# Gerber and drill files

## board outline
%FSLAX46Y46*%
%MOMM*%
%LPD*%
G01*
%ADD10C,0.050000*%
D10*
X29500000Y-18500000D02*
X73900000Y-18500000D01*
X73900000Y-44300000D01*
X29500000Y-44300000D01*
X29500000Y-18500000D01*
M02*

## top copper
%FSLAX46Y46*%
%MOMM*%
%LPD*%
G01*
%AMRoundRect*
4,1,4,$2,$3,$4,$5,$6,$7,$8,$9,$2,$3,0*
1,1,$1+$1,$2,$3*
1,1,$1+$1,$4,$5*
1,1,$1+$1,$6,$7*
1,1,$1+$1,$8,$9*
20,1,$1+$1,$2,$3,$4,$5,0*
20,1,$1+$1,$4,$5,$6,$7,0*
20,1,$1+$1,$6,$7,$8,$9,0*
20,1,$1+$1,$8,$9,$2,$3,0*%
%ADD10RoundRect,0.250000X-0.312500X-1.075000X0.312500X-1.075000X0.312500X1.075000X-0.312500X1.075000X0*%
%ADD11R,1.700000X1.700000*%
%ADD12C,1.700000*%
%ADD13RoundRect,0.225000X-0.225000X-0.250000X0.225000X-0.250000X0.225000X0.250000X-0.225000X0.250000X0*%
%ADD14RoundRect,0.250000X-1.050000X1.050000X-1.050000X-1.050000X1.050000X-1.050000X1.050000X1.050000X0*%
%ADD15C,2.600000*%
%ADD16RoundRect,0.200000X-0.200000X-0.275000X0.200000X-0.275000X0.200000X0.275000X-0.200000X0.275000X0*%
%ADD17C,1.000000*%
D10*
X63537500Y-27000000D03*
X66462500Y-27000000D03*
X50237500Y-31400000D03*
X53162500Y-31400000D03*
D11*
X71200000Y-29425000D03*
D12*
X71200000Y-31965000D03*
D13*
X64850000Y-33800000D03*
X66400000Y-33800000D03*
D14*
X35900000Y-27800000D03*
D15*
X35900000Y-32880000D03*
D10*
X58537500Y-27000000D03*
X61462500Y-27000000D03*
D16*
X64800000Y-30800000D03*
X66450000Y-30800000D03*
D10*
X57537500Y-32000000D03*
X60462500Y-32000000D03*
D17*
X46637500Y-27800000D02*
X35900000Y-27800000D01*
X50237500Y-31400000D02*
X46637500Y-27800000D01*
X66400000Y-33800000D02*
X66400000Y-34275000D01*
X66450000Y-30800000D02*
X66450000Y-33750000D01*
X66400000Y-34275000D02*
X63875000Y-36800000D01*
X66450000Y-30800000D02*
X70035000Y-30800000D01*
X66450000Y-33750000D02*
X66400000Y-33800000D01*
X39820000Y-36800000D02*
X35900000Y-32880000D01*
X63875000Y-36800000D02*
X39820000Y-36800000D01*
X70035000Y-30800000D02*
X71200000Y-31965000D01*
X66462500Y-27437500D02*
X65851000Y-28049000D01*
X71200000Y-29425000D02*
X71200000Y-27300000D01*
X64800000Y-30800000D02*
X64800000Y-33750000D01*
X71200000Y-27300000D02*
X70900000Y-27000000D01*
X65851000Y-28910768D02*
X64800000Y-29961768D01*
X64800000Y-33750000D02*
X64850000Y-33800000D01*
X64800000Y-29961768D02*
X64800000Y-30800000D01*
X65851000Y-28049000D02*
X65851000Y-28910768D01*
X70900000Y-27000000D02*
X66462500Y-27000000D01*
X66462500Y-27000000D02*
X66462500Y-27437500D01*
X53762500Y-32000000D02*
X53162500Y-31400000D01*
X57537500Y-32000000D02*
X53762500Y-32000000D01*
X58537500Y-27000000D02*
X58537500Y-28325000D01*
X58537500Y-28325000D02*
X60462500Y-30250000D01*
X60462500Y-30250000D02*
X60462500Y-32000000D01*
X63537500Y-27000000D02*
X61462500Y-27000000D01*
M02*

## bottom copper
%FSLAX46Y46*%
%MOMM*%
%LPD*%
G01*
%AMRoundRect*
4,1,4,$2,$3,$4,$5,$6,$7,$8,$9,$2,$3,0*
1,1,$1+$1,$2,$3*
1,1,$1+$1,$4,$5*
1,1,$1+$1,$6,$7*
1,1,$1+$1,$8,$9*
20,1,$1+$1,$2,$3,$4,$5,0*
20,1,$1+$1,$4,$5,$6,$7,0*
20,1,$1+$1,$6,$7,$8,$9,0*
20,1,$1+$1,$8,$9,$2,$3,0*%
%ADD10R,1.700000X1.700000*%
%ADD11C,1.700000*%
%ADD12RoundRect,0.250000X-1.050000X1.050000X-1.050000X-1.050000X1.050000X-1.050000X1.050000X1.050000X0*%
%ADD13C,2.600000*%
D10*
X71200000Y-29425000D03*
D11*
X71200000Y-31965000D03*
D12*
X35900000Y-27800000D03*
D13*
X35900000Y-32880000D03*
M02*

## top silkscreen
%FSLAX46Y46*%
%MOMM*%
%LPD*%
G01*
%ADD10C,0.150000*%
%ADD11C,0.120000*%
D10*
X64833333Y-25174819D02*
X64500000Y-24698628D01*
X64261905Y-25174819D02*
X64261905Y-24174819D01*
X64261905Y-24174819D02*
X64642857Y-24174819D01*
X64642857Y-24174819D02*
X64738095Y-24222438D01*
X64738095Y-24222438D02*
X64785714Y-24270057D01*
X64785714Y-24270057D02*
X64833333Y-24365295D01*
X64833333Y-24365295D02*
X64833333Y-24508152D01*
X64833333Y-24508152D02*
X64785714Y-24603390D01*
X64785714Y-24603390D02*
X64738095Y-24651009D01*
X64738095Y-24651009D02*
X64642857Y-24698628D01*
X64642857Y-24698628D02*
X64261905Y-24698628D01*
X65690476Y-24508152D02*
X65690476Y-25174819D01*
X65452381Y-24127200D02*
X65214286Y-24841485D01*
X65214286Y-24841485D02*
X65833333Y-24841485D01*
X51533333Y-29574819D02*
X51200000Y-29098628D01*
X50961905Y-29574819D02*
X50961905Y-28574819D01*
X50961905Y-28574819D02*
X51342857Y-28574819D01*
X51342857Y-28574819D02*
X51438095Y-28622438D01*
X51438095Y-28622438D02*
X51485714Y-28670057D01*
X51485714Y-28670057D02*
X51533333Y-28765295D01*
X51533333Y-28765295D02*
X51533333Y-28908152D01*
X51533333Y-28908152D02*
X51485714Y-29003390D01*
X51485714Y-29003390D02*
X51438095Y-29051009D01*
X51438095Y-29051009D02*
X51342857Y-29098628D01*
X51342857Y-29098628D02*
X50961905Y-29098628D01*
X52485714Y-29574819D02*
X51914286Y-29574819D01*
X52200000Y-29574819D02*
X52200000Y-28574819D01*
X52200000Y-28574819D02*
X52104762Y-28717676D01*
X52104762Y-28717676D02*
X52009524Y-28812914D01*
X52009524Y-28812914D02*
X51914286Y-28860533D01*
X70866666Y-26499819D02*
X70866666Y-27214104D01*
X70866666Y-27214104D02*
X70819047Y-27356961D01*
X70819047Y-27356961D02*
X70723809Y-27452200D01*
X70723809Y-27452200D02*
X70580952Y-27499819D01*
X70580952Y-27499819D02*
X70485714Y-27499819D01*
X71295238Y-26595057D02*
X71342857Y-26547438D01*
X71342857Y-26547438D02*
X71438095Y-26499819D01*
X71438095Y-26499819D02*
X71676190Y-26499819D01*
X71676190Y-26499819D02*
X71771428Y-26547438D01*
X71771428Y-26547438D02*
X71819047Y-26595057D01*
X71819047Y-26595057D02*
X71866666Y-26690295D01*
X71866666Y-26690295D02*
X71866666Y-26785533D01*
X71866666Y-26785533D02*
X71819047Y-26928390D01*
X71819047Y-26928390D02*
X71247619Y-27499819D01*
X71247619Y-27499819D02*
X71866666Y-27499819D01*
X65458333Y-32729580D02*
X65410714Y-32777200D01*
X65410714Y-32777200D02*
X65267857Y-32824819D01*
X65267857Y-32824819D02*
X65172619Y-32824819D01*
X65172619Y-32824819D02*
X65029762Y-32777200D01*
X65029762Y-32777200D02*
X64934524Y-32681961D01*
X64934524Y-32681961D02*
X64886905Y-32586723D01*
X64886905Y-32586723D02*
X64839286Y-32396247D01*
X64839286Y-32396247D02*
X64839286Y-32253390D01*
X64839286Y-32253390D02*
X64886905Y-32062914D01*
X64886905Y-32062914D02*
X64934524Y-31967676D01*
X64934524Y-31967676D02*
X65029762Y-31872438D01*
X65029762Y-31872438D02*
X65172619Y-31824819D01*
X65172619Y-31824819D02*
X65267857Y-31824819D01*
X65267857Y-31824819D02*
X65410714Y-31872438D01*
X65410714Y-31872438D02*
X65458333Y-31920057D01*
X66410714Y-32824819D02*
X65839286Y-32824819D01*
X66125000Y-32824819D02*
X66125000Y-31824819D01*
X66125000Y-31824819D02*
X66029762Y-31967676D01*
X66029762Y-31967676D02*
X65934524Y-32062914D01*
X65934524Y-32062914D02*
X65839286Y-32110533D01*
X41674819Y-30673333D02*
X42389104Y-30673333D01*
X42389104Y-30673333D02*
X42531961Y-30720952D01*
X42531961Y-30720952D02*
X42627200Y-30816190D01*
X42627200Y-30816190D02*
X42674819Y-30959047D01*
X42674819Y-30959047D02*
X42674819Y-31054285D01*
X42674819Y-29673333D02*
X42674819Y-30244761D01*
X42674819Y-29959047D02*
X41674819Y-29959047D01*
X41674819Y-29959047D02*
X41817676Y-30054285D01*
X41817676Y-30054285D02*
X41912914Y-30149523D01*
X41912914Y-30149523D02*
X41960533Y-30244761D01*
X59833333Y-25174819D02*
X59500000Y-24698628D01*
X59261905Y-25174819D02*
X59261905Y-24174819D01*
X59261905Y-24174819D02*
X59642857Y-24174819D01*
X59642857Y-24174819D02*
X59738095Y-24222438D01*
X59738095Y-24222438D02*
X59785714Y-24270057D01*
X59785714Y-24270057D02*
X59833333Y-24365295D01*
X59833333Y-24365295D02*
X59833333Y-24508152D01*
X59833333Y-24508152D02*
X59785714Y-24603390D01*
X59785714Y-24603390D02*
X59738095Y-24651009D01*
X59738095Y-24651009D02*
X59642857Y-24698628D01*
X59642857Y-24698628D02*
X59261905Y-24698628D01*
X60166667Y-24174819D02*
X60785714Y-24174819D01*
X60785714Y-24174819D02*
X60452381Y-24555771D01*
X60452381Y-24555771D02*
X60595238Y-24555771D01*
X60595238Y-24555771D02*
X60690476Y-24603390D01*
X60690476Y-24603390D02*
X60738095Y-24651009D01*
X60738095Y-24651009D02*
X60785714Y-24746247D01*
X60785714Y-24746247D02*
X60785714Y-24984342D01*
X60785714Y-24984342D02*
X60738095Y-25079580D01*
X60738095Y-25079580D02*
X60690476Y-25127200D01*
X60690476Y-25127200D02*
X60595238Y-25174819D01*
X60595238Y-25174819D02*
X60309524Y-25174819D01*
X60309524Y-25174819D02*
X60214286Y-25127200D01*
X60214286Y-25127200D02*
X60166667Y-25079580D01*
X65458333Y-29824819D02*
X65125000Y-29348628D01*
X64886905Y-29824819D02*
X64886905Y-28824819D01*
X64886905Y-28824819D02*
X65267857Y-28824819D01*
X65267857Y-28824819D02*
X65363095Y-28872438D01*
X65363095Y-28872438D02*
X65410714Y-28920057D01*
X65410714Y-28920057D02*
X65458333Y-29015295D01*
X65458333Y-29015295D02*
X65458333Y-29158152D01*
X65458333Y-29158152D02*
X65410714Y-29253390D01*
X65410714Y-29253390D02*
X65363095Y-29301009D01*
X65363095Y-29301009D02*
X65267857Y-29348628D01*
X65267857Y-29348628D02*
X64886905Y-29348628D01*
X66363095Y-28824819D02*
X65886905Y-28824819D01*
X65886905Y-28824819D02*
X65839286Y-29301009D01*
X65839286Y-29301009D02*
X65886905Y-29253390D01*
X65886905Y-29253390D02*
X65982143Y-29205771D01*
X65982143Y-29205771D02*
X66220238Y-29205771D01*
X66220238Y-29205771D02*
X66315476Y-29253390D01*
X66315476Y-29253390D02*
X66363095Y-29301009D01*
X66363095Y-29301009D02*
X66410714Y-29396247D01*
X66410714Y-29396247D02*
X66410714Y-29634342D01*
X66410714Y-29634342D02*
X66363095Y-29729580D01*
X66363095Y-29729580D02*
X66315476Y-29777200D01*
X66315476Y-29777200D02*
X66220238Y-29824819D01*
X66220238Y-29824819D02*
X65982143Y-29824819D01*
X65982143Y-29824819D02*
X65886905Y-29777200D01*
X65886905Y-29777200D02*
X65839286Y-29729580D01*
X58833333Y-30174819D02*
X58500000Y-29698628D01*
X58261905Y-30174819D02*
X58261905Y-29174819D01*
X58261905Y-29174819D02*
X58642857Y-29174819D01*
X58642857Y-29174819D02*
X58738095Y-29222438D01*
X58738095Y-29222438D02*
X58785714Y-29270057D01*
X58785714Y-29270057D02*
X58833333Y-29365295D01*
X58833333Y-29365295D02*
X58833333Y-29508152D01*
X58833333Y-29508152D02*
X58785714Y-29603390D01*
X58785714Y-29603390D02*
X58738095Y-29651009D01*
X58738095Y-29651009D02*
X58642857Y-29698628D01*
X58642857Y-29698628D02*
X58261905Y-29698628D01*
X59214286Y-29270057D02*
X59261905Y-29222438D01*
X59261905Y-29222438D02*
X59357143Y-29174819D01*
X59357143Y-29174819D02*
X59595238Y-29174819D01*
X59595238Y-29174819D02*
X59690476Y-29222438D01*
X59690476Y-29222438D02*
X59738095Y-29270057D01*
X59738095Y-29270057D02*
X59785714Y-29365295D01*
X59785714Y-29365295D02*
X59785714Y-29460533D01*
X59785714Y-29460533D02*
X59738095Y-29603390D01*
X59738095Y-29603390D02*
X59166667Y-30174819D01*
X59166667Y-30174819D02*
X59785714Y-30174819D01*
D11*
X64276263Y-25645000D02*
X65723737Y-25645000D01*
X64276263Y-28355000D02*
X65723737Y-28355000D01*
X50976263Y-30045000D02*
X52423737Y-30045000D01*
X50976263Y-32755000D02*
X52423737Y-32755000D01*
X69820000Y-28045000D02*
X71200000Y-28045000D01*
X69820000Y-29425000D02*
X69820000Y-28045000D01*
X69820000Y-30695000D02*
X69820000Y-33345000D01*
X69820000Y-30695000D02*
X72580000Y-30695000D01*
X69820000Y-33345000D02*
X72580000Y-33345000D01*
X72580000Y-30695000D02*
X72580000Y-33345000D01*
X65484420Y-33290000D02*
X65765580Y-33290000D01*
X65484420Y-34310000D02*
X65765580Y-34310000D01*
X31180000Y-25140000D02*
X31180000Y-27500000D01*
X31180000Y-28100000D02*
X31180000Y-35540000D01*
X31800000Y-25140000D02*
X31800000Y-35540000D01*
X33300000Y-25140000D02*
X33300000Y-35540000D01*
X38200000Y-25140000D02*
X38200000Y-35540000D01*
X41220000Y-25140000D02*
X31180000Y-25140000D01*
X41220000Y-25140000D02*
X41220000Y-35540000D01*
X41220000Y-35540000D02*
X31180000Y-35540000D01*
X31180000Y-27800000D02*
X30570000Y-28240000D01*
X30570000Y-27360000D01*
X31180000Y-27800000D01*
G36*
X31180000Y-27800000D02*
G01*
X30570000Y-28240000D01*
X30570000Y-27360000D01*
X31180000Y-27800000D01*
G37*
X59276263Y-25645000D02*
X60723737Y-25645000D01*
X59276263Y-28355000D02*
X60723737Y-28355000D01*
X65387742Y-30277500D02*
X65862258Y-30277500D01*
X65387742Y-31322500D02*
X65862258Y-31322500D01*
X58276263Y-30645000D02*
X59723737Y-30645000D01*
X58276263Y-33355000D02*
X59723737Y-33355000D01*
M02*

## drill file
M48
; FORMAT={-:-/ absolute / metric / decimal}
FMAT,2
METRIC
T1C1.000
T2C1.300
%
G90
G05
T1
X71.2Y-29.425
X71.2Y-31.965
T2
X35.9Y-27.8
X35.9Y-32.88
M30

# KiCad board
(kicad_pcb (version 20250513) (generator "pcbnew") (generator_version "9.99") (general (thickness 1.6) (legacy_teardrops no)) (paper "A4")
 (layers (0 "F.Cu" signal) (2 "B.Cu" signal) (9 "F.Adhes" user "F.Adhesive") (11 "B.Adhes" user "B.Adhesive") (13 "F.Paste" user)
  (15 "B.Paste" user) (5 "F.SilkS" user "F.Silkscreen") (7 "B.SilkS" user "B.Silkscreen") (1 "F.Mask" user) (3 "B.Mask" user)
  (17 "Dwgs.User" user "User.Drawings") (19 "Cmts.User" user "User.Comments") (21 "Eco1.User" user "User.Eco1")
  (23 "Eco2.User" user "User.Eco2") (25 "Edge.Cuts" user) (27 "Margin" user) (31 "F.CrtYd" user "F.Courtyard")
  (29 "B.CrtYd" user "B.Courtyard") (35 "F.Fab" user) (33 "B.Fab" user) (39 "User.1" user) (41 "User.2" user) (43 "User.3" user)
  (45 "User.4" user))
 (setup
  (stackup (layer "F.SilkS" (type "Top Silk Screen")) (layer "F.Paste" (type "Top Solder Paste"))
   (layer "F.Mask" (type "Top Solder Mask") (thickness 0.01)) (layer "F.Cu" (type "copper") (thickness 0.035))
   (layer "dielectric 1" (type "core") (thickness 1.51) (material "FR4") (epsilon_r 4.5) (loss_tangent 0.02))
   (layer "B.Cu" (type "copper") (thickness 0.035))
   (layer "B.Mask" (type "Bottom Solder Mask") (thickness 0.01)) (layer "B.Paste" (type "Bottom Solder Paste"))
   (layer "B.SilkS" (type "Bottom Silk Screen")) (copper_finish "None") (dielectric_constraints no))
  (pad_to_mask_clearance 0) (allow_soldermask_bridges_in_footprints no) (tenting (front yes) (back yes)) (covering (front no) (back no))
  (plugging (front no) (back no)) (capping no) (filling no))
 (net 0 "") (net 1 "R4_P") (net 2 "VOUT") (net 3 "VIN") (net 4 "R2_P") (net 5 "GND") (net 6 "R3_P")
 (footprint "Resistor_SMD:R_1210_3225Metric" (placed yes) (layer "F.Cu") (at 65 27)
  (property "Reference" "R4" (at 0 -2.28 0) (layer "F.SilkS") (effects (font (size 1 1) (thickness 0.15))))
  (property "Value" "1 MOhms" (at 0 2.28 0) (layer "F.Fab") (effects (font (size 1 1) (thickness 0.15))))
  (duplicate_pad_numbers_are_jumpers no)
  (fp_line (start -0.723737 -1.355) (end 0.723737 -1.355) (stroke (width 0.12) (type solid)) (layer "F.SilkS"))
  (fp_line (start -0.723737 1.355) (end 0.723737 1.355) (stroke (width 0.12) (type solid)) (layer "F.SilkS"))
  (pad "1" smd roundrect (at -1.4625 0) (size 1.125 2.65) (layers "F.Cu" "F.Mask" "F.Paste") (roundrect_rratio 0.222222) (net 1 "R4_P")
   (tenting (front none) (back none)))
  (pad "2" smd roundrect (at 1.4625 0) (size 1.125 2.65) (layers "F.Cu" "F.Mask" "F.Paste") (roundrect_rratio 0.222222) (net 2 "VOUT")
   (tenting (front none) (back none))))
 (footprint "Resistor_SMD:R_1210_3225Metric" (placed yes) (layer "F.Cu") (at 51.7 31.4)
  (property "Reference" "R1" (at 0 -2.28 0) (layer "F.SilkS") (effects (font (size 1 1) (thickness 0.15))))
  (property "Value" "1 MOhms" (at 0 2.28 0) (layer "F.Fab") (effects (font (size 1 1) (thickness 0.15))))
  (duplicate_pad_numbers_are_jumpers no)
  (fp_line (start -0.723737 -1.355) (end 0.723737 -1.355) (stroke (width 0.12) (type solid)) (layer "F.SilkS"))
  (fp_line (start -0.723737 1.355) (end 0.723737 1.355) (stroke (width 0.12) (type solid)) (layer "F.SilkS"))
  (pad "1" smd roundrect (at -1.4625 0) (size 1.125 2.65) (layers "F.Cu" "F.Mask" "F.Paste") (roundrect_rratio 0.222222) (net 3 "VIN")
   (tenting (front none) (back none)))
  (pad "2" smd roundrect (at 1.4625 0) (size 1.125 2.65) (layers "F.Cu" "F.Mask" "F.Paste") (roundrect_rratio 0.222222) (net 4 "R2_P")
   (tenting (front none) (back none))))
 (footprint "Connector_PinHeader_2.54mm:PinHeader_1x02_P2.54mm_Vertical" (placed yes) (layer "F.Cu") (at 71.2 29.425)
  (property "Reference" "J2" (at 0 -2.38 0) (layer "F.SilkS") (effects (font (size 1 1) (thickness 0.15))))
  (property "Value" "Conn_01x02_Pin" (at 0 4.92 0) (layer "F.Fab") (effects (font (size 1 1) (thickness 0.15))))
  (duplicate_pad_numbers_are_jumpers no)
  (fp_line (start -1.38 -1.38) (end 0 -1.38) (stroke (width 0.12) (type solid)) (layer "F.SilkS"))
  (fp_line (start -1.38 0) (end -1.38 -1.38) (stroke (width 0.12) (type solid)) (layer "F.SilkS"))
  (fp_line (start -1.38 1.27) (end -1.38 3.92) (stroke (width 0.12) (type solid)) (layer "F.SilkS"))
  (fp_line (start -1.38 1.27) (end 1.38 1.27) (stroke (width 0.12) (type solid)) (layer "F.SilkS"))
  (fp_line (start -1.38 3.92) (end 1.38 3.92) (stroke (width 0.12) (type solid)) (layer "F.SilkS"))
  (fp_line (start 1.38 1.27) (end 1.38 3.92) (stroke (width 0.12) (type solid)) (layer "F.SilkS"))
  (pad "1" thru_hole rect (at 0 0) (size 1.7 1.7) (drill 1) (layers "*.Cu" "*.Mask") (remove_unused_layers no) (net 2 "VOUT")
   (tenting (front none) (back none)))
  (pad "2" thru_hole circle (at 0 2.54) (size 1.7 1.7) (drill 1) (layers "*.Cu" "*.Mask") (remove_unused_layers no) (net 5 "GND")
   (tenting (front none) (back none))))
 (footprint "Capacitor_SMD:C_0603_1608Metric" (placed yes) (layer "F.Cu") (at 65.625 33.8)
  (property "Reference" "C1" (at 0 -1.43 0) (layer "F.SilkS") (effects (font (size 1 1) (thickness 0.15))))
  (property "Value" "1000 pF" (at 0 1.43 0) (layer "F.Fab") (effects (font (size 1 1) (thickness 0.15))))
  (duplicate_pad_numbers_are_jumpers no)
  (fp_line (start -0.14058 -0.51) (end 0.14058 -0.51) (stroke (width 0.12) (type solid)) (layer "F.SilkS"))
  (fp_line (start -0.14058 0.51) (end 0.14058 0.51) (stroke (width 0.12) (type solid)) (layer "F.SilkS"))
  (pad "1" smd roundrect (at -0.775 0) (size 0.9 0.95) (layers "F.Cu" "F.Mask" "F.Paste") (roundrect_rratio 0.25) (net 2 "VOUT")
   (tenting (front none) (back none)))
  (pad "2" smd roundrect (at 0.775 0) (size 0.9 0.95) (layers "F.Cu" "F.Mask" "F.Paste") (roundrect_rratio 0.25) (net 5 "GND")
   (tenting (front none) (back none))))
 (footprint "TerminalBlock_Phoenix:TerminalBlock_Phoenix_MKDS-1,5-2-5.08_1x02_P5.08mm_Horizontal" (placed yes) (layer "F.Cu")
  (at 35.9 27.8 -90)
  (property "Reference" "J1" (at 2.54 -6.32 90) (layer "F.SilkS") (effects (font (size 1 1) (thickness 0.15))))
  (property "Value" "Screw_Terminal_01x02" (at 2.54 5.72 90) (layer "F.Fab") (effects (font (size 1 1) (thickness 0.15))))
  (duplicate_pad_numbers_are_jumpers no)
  (fp_line (start -2.66 4.72) (end -0.3 4.72) (stroke (width 0.12) (type solid)) (layer "F.SilkS"))
  (fp_line (start 0.3 4.72) (end 7.74 4.72) (stroke (width 0.12) (type solid)) (layer "F.SilkS"))
  (fp_line (start -2.66 4.1) (end 7.74 4.1) (stroke (width 0.12) (type solid)) (layer "F.SilkS"))
  (fp_line (start -2.66 2.6) (end 7.74 2.6) (stroke (width 0.12) (type solid)) (layer "F.SilkS"))
  (fp_line (start -2.66 -2.3) (end 7.74 -2.3) (stroke (width 0.12) (type solid)) (layer "F.SilkS"))
  (fp_line (start -2.66 -5.32) (end -2.66 4.72) (stroke (width 0.12) (type solid)) (layer "F.SilkS"))
  (fp_line (start -2.66 -5.32) (end 7.74 -5.32) (stroke (width 0.12) (type solid)) (layer "F.SilkS"))
  (fp_line (start 7.74 -5.32) (end 7.74 4.72) (stroke (width 0.12) (type solid)) (layer "F.SilkS"))
  (fp_poly (pts (xy 0 4.72) (xy 0.44 5.33) (xy -0.44 5.33)) (stroke (width 0.12) (type solid)) (fill yes) (layer "F.SilkS"))
  (pad "1" thru_hole roundrect (at 0 0 270) (size 2.6 2.6) (drill 1.3) (layers "*.Cu" "*.Mask") (remove_unused_layers no)
   (roundrect_rratio 0.096154) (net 3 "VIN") (tenting (front none) (back none)))
  (pad "2" thru_hole circle (at 5.08 0 270) (size 2.6 2.6) (drill 1.3) (layers "*.Cu" "*.Mask") (remove_unused_layers no) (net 5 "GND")
   (tenting (front none) (back none))))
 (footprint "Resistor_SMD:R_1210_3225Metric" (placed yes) (layer "F.Cu") (at 60 27)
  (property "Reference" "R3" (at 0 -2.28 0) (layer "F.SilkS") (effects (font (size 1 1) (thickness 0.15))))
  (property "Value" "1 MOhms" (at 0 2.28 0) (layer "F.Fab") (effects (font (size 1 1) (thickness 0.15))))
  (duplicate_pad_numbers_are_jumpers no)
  (fp_line (start -0.723737 -1.355) (end 0.723737 -1.355) (stroke (width 0.12) (type solid)) (layer "F.SilkS"))
  (fp_line (start -0.723737 1.355) (end 0.723737 1.355) (stroke (width 0.12) (type solid)) (layer "F.SilkS"))
  (pad "1" smd roundrect (at -1.4625 0) (size 1.125 2.65) (layers "F.Cu" "F.Mask" "F.Paste") (roundrect_rratio 0.222222) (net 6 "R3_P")
   (tenting (front none) (back none)))
  (pad "2" smd roundrect (at 1.4625 0) (size 1.125 2.65) (layers "F.Cu" "F.Mask" "F.Paste") (roundrect_rratio 0.222222) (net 1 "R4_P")
   (tenting (front none) (back none))))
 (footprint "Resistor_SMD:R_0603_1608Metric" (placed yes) (layer "F.Cu") (at 65.625 30.8)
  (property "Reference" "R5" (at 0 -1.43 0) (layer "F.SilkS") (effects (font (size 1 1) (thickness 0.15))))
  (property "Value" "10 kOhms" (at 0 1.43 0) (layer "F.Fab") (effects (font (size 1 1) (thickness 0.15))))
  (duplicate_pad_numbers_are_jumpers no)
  (fp_line (start -0.237258 -0.5225) (end 0.237258 -0.5225) (stroke (width 0.12) (type solid)) (layer "F.SilkS"))
  (fp_line (start -0.237258 0.5225) (end 0.237258 0.5225) (stroke (width 0.12) (type solid)) (layer "F.SilkS"))
  (pad "1" smd roundrect (at -0.825 0) (size 0.8 0.95) (layers "F.Cu" "F.Mask" "F.Paste") (roundrect_rratio 0.25) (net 2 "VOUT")
   (tenting (front none) (back none)))
  (pad "2" smd roundrect (at 0.825 0) (size 0.8 0.95) (layers "F.Cu" "F.Mask" "F.Paste") (roundrect_rratio 0.25) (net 5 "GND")
   (tenting (front none) (back none))))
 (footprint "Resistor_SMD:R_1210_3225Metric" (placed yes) (layer "F.Cu") (at 59 32)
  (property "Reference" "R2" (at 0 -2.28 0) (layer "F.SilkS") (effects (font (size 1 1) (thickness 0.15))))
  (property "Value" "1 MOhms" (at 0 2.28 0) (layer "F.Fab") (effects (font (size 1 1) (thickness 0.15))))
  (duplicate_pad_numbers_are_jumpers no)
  (fp_line (start -0.723737 -1.355) (end 0.723737 -1.355) (stroke (width 0.12) (type solid)) (layer "F.SilkS"))
  (fp_line (start -0.723737 1.355) (end 0.723737 1.355) (stroke (width 0.12) (type solid)) (layer "F.SilkS"))
  (pad "1" smd roundrect (at -1.4625 0) (size 1.125 2.65) (layers "F.Cu" "F.Mask" "F.Paste") (roundrect_rratio 0.222222) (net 4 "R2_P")
   (tenting (front none) (back none)))
  (pad "2" smd roundrect (at 1.4625 0) (size 1.125 2.65) (layers "F.Cu" "F.Mask" "F.Paste") (roundrect_rratio 0.222222) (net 6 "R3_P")
   (tenting (front none) (back none))))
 (gr_rect (start 29.5 18.5) (end 73.9 44.3) (stroke (width 0.05) (type default)) (fill no) (layer "Edge.Cuts"))
 (segment (start 46.6375 27.8) (end 35.9 27.8) (width 1) (layer "F.Cu") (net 3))
 (segment (start 50.2375 31.4) (end 46.6375 27.8) (width 1) (layer "F.Cu") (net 3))
 (segment (start 66.4 33.8) (end 66.4 34.275) (width 1) (layer "F.Cu") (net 5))
 (segment (start 66.45 30.8) (end 66.45 33.75) (width 1) (layer "F.Cu") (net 5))
 (segment (start 66.4 34.275) (end 63.875 36.8) (width 1) (layer "F.Cu") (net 5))
 (segment (start 66.45 30.8) (end 70.035 30.8) (width 1) (layer "F.Cu") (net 5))
 (segment (start 66.45 33.75) (end 66.4 33.8) (width 1) (layer "F.Cu") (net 5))
 (segment (start 39.82 36.8) (end 35.9 32.88) (width 1) (layer "F.Cu") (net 5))
 (segment (start 63.875 36.8) (end 39.82 36.8) (width 1) (layer "F.Cu") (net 5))
 (segment (start 70.035 30.8) (end 71.2 31.965) (width 1) (layer "F.Cu") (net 5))
 (segment (start 66.4625 27.4375) (end 65.851 28.049) (width 1) (layer "F.Cu") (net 2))
 (segment (start 71.2 29.425) (end 71.2 27.3) (width 1) (layer "F.Cu") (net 2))
 (segment (start 64.8 30.8) (end 64.8 33.75) (width 1) (layer "F.Cu") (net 2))
 (segment (start 71.2 27.3) (end 70.9 27) (width 1) (layer "F.Cu") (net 2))
 (segment (start 65.851 28.910768) (end 64.8 29.961768) (width 1) (layer "F.Cu") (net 2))
 (segment (start 64.8 33.75) (end 64.85 33.8) (width 1) (layer "F.Cu") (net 2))
 (segment (start 64.8 29.961768) (end 64.8 30.8) (width 1) (layer "F.Cu") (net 2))
 (segment (start 65.851 28.049) (end 65.851 28.910768) (width 1) (layer "F.Cu") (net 2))
 (segment (start 70.9 27) (end 66.4625 27) (width 1) (layer "F.Cu") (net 2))
 (segment (start 66.4625 27) (end 66.4625 27.4375) (width 1) (layer "F.Cu") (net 2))
 (segment (start 53.7625 32) (end 53.1625 31.4) (width 1) (layer "F.Cu") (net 4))
 (segment (start 57.5375 32) (end 53.7625 32) (width 1) (layer "F.Cu") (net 4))
 (segment (start 58.5375 27) (end 58.5375 28.325) (width 1) (layer "F.Cu") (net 6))
 (segment (start 58.5375 28.325) (end 60.4625 30.25) (width 1) (layer "F.Cu") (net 6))
 (segment (start 60.4625 30.25) (end 60.4625 32) (width 1) (layer "F.Cu") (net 6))
 (segment (start 63.5375 27) (end 61.4625 27) (width 1) (layer "F.Cu") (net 1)))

